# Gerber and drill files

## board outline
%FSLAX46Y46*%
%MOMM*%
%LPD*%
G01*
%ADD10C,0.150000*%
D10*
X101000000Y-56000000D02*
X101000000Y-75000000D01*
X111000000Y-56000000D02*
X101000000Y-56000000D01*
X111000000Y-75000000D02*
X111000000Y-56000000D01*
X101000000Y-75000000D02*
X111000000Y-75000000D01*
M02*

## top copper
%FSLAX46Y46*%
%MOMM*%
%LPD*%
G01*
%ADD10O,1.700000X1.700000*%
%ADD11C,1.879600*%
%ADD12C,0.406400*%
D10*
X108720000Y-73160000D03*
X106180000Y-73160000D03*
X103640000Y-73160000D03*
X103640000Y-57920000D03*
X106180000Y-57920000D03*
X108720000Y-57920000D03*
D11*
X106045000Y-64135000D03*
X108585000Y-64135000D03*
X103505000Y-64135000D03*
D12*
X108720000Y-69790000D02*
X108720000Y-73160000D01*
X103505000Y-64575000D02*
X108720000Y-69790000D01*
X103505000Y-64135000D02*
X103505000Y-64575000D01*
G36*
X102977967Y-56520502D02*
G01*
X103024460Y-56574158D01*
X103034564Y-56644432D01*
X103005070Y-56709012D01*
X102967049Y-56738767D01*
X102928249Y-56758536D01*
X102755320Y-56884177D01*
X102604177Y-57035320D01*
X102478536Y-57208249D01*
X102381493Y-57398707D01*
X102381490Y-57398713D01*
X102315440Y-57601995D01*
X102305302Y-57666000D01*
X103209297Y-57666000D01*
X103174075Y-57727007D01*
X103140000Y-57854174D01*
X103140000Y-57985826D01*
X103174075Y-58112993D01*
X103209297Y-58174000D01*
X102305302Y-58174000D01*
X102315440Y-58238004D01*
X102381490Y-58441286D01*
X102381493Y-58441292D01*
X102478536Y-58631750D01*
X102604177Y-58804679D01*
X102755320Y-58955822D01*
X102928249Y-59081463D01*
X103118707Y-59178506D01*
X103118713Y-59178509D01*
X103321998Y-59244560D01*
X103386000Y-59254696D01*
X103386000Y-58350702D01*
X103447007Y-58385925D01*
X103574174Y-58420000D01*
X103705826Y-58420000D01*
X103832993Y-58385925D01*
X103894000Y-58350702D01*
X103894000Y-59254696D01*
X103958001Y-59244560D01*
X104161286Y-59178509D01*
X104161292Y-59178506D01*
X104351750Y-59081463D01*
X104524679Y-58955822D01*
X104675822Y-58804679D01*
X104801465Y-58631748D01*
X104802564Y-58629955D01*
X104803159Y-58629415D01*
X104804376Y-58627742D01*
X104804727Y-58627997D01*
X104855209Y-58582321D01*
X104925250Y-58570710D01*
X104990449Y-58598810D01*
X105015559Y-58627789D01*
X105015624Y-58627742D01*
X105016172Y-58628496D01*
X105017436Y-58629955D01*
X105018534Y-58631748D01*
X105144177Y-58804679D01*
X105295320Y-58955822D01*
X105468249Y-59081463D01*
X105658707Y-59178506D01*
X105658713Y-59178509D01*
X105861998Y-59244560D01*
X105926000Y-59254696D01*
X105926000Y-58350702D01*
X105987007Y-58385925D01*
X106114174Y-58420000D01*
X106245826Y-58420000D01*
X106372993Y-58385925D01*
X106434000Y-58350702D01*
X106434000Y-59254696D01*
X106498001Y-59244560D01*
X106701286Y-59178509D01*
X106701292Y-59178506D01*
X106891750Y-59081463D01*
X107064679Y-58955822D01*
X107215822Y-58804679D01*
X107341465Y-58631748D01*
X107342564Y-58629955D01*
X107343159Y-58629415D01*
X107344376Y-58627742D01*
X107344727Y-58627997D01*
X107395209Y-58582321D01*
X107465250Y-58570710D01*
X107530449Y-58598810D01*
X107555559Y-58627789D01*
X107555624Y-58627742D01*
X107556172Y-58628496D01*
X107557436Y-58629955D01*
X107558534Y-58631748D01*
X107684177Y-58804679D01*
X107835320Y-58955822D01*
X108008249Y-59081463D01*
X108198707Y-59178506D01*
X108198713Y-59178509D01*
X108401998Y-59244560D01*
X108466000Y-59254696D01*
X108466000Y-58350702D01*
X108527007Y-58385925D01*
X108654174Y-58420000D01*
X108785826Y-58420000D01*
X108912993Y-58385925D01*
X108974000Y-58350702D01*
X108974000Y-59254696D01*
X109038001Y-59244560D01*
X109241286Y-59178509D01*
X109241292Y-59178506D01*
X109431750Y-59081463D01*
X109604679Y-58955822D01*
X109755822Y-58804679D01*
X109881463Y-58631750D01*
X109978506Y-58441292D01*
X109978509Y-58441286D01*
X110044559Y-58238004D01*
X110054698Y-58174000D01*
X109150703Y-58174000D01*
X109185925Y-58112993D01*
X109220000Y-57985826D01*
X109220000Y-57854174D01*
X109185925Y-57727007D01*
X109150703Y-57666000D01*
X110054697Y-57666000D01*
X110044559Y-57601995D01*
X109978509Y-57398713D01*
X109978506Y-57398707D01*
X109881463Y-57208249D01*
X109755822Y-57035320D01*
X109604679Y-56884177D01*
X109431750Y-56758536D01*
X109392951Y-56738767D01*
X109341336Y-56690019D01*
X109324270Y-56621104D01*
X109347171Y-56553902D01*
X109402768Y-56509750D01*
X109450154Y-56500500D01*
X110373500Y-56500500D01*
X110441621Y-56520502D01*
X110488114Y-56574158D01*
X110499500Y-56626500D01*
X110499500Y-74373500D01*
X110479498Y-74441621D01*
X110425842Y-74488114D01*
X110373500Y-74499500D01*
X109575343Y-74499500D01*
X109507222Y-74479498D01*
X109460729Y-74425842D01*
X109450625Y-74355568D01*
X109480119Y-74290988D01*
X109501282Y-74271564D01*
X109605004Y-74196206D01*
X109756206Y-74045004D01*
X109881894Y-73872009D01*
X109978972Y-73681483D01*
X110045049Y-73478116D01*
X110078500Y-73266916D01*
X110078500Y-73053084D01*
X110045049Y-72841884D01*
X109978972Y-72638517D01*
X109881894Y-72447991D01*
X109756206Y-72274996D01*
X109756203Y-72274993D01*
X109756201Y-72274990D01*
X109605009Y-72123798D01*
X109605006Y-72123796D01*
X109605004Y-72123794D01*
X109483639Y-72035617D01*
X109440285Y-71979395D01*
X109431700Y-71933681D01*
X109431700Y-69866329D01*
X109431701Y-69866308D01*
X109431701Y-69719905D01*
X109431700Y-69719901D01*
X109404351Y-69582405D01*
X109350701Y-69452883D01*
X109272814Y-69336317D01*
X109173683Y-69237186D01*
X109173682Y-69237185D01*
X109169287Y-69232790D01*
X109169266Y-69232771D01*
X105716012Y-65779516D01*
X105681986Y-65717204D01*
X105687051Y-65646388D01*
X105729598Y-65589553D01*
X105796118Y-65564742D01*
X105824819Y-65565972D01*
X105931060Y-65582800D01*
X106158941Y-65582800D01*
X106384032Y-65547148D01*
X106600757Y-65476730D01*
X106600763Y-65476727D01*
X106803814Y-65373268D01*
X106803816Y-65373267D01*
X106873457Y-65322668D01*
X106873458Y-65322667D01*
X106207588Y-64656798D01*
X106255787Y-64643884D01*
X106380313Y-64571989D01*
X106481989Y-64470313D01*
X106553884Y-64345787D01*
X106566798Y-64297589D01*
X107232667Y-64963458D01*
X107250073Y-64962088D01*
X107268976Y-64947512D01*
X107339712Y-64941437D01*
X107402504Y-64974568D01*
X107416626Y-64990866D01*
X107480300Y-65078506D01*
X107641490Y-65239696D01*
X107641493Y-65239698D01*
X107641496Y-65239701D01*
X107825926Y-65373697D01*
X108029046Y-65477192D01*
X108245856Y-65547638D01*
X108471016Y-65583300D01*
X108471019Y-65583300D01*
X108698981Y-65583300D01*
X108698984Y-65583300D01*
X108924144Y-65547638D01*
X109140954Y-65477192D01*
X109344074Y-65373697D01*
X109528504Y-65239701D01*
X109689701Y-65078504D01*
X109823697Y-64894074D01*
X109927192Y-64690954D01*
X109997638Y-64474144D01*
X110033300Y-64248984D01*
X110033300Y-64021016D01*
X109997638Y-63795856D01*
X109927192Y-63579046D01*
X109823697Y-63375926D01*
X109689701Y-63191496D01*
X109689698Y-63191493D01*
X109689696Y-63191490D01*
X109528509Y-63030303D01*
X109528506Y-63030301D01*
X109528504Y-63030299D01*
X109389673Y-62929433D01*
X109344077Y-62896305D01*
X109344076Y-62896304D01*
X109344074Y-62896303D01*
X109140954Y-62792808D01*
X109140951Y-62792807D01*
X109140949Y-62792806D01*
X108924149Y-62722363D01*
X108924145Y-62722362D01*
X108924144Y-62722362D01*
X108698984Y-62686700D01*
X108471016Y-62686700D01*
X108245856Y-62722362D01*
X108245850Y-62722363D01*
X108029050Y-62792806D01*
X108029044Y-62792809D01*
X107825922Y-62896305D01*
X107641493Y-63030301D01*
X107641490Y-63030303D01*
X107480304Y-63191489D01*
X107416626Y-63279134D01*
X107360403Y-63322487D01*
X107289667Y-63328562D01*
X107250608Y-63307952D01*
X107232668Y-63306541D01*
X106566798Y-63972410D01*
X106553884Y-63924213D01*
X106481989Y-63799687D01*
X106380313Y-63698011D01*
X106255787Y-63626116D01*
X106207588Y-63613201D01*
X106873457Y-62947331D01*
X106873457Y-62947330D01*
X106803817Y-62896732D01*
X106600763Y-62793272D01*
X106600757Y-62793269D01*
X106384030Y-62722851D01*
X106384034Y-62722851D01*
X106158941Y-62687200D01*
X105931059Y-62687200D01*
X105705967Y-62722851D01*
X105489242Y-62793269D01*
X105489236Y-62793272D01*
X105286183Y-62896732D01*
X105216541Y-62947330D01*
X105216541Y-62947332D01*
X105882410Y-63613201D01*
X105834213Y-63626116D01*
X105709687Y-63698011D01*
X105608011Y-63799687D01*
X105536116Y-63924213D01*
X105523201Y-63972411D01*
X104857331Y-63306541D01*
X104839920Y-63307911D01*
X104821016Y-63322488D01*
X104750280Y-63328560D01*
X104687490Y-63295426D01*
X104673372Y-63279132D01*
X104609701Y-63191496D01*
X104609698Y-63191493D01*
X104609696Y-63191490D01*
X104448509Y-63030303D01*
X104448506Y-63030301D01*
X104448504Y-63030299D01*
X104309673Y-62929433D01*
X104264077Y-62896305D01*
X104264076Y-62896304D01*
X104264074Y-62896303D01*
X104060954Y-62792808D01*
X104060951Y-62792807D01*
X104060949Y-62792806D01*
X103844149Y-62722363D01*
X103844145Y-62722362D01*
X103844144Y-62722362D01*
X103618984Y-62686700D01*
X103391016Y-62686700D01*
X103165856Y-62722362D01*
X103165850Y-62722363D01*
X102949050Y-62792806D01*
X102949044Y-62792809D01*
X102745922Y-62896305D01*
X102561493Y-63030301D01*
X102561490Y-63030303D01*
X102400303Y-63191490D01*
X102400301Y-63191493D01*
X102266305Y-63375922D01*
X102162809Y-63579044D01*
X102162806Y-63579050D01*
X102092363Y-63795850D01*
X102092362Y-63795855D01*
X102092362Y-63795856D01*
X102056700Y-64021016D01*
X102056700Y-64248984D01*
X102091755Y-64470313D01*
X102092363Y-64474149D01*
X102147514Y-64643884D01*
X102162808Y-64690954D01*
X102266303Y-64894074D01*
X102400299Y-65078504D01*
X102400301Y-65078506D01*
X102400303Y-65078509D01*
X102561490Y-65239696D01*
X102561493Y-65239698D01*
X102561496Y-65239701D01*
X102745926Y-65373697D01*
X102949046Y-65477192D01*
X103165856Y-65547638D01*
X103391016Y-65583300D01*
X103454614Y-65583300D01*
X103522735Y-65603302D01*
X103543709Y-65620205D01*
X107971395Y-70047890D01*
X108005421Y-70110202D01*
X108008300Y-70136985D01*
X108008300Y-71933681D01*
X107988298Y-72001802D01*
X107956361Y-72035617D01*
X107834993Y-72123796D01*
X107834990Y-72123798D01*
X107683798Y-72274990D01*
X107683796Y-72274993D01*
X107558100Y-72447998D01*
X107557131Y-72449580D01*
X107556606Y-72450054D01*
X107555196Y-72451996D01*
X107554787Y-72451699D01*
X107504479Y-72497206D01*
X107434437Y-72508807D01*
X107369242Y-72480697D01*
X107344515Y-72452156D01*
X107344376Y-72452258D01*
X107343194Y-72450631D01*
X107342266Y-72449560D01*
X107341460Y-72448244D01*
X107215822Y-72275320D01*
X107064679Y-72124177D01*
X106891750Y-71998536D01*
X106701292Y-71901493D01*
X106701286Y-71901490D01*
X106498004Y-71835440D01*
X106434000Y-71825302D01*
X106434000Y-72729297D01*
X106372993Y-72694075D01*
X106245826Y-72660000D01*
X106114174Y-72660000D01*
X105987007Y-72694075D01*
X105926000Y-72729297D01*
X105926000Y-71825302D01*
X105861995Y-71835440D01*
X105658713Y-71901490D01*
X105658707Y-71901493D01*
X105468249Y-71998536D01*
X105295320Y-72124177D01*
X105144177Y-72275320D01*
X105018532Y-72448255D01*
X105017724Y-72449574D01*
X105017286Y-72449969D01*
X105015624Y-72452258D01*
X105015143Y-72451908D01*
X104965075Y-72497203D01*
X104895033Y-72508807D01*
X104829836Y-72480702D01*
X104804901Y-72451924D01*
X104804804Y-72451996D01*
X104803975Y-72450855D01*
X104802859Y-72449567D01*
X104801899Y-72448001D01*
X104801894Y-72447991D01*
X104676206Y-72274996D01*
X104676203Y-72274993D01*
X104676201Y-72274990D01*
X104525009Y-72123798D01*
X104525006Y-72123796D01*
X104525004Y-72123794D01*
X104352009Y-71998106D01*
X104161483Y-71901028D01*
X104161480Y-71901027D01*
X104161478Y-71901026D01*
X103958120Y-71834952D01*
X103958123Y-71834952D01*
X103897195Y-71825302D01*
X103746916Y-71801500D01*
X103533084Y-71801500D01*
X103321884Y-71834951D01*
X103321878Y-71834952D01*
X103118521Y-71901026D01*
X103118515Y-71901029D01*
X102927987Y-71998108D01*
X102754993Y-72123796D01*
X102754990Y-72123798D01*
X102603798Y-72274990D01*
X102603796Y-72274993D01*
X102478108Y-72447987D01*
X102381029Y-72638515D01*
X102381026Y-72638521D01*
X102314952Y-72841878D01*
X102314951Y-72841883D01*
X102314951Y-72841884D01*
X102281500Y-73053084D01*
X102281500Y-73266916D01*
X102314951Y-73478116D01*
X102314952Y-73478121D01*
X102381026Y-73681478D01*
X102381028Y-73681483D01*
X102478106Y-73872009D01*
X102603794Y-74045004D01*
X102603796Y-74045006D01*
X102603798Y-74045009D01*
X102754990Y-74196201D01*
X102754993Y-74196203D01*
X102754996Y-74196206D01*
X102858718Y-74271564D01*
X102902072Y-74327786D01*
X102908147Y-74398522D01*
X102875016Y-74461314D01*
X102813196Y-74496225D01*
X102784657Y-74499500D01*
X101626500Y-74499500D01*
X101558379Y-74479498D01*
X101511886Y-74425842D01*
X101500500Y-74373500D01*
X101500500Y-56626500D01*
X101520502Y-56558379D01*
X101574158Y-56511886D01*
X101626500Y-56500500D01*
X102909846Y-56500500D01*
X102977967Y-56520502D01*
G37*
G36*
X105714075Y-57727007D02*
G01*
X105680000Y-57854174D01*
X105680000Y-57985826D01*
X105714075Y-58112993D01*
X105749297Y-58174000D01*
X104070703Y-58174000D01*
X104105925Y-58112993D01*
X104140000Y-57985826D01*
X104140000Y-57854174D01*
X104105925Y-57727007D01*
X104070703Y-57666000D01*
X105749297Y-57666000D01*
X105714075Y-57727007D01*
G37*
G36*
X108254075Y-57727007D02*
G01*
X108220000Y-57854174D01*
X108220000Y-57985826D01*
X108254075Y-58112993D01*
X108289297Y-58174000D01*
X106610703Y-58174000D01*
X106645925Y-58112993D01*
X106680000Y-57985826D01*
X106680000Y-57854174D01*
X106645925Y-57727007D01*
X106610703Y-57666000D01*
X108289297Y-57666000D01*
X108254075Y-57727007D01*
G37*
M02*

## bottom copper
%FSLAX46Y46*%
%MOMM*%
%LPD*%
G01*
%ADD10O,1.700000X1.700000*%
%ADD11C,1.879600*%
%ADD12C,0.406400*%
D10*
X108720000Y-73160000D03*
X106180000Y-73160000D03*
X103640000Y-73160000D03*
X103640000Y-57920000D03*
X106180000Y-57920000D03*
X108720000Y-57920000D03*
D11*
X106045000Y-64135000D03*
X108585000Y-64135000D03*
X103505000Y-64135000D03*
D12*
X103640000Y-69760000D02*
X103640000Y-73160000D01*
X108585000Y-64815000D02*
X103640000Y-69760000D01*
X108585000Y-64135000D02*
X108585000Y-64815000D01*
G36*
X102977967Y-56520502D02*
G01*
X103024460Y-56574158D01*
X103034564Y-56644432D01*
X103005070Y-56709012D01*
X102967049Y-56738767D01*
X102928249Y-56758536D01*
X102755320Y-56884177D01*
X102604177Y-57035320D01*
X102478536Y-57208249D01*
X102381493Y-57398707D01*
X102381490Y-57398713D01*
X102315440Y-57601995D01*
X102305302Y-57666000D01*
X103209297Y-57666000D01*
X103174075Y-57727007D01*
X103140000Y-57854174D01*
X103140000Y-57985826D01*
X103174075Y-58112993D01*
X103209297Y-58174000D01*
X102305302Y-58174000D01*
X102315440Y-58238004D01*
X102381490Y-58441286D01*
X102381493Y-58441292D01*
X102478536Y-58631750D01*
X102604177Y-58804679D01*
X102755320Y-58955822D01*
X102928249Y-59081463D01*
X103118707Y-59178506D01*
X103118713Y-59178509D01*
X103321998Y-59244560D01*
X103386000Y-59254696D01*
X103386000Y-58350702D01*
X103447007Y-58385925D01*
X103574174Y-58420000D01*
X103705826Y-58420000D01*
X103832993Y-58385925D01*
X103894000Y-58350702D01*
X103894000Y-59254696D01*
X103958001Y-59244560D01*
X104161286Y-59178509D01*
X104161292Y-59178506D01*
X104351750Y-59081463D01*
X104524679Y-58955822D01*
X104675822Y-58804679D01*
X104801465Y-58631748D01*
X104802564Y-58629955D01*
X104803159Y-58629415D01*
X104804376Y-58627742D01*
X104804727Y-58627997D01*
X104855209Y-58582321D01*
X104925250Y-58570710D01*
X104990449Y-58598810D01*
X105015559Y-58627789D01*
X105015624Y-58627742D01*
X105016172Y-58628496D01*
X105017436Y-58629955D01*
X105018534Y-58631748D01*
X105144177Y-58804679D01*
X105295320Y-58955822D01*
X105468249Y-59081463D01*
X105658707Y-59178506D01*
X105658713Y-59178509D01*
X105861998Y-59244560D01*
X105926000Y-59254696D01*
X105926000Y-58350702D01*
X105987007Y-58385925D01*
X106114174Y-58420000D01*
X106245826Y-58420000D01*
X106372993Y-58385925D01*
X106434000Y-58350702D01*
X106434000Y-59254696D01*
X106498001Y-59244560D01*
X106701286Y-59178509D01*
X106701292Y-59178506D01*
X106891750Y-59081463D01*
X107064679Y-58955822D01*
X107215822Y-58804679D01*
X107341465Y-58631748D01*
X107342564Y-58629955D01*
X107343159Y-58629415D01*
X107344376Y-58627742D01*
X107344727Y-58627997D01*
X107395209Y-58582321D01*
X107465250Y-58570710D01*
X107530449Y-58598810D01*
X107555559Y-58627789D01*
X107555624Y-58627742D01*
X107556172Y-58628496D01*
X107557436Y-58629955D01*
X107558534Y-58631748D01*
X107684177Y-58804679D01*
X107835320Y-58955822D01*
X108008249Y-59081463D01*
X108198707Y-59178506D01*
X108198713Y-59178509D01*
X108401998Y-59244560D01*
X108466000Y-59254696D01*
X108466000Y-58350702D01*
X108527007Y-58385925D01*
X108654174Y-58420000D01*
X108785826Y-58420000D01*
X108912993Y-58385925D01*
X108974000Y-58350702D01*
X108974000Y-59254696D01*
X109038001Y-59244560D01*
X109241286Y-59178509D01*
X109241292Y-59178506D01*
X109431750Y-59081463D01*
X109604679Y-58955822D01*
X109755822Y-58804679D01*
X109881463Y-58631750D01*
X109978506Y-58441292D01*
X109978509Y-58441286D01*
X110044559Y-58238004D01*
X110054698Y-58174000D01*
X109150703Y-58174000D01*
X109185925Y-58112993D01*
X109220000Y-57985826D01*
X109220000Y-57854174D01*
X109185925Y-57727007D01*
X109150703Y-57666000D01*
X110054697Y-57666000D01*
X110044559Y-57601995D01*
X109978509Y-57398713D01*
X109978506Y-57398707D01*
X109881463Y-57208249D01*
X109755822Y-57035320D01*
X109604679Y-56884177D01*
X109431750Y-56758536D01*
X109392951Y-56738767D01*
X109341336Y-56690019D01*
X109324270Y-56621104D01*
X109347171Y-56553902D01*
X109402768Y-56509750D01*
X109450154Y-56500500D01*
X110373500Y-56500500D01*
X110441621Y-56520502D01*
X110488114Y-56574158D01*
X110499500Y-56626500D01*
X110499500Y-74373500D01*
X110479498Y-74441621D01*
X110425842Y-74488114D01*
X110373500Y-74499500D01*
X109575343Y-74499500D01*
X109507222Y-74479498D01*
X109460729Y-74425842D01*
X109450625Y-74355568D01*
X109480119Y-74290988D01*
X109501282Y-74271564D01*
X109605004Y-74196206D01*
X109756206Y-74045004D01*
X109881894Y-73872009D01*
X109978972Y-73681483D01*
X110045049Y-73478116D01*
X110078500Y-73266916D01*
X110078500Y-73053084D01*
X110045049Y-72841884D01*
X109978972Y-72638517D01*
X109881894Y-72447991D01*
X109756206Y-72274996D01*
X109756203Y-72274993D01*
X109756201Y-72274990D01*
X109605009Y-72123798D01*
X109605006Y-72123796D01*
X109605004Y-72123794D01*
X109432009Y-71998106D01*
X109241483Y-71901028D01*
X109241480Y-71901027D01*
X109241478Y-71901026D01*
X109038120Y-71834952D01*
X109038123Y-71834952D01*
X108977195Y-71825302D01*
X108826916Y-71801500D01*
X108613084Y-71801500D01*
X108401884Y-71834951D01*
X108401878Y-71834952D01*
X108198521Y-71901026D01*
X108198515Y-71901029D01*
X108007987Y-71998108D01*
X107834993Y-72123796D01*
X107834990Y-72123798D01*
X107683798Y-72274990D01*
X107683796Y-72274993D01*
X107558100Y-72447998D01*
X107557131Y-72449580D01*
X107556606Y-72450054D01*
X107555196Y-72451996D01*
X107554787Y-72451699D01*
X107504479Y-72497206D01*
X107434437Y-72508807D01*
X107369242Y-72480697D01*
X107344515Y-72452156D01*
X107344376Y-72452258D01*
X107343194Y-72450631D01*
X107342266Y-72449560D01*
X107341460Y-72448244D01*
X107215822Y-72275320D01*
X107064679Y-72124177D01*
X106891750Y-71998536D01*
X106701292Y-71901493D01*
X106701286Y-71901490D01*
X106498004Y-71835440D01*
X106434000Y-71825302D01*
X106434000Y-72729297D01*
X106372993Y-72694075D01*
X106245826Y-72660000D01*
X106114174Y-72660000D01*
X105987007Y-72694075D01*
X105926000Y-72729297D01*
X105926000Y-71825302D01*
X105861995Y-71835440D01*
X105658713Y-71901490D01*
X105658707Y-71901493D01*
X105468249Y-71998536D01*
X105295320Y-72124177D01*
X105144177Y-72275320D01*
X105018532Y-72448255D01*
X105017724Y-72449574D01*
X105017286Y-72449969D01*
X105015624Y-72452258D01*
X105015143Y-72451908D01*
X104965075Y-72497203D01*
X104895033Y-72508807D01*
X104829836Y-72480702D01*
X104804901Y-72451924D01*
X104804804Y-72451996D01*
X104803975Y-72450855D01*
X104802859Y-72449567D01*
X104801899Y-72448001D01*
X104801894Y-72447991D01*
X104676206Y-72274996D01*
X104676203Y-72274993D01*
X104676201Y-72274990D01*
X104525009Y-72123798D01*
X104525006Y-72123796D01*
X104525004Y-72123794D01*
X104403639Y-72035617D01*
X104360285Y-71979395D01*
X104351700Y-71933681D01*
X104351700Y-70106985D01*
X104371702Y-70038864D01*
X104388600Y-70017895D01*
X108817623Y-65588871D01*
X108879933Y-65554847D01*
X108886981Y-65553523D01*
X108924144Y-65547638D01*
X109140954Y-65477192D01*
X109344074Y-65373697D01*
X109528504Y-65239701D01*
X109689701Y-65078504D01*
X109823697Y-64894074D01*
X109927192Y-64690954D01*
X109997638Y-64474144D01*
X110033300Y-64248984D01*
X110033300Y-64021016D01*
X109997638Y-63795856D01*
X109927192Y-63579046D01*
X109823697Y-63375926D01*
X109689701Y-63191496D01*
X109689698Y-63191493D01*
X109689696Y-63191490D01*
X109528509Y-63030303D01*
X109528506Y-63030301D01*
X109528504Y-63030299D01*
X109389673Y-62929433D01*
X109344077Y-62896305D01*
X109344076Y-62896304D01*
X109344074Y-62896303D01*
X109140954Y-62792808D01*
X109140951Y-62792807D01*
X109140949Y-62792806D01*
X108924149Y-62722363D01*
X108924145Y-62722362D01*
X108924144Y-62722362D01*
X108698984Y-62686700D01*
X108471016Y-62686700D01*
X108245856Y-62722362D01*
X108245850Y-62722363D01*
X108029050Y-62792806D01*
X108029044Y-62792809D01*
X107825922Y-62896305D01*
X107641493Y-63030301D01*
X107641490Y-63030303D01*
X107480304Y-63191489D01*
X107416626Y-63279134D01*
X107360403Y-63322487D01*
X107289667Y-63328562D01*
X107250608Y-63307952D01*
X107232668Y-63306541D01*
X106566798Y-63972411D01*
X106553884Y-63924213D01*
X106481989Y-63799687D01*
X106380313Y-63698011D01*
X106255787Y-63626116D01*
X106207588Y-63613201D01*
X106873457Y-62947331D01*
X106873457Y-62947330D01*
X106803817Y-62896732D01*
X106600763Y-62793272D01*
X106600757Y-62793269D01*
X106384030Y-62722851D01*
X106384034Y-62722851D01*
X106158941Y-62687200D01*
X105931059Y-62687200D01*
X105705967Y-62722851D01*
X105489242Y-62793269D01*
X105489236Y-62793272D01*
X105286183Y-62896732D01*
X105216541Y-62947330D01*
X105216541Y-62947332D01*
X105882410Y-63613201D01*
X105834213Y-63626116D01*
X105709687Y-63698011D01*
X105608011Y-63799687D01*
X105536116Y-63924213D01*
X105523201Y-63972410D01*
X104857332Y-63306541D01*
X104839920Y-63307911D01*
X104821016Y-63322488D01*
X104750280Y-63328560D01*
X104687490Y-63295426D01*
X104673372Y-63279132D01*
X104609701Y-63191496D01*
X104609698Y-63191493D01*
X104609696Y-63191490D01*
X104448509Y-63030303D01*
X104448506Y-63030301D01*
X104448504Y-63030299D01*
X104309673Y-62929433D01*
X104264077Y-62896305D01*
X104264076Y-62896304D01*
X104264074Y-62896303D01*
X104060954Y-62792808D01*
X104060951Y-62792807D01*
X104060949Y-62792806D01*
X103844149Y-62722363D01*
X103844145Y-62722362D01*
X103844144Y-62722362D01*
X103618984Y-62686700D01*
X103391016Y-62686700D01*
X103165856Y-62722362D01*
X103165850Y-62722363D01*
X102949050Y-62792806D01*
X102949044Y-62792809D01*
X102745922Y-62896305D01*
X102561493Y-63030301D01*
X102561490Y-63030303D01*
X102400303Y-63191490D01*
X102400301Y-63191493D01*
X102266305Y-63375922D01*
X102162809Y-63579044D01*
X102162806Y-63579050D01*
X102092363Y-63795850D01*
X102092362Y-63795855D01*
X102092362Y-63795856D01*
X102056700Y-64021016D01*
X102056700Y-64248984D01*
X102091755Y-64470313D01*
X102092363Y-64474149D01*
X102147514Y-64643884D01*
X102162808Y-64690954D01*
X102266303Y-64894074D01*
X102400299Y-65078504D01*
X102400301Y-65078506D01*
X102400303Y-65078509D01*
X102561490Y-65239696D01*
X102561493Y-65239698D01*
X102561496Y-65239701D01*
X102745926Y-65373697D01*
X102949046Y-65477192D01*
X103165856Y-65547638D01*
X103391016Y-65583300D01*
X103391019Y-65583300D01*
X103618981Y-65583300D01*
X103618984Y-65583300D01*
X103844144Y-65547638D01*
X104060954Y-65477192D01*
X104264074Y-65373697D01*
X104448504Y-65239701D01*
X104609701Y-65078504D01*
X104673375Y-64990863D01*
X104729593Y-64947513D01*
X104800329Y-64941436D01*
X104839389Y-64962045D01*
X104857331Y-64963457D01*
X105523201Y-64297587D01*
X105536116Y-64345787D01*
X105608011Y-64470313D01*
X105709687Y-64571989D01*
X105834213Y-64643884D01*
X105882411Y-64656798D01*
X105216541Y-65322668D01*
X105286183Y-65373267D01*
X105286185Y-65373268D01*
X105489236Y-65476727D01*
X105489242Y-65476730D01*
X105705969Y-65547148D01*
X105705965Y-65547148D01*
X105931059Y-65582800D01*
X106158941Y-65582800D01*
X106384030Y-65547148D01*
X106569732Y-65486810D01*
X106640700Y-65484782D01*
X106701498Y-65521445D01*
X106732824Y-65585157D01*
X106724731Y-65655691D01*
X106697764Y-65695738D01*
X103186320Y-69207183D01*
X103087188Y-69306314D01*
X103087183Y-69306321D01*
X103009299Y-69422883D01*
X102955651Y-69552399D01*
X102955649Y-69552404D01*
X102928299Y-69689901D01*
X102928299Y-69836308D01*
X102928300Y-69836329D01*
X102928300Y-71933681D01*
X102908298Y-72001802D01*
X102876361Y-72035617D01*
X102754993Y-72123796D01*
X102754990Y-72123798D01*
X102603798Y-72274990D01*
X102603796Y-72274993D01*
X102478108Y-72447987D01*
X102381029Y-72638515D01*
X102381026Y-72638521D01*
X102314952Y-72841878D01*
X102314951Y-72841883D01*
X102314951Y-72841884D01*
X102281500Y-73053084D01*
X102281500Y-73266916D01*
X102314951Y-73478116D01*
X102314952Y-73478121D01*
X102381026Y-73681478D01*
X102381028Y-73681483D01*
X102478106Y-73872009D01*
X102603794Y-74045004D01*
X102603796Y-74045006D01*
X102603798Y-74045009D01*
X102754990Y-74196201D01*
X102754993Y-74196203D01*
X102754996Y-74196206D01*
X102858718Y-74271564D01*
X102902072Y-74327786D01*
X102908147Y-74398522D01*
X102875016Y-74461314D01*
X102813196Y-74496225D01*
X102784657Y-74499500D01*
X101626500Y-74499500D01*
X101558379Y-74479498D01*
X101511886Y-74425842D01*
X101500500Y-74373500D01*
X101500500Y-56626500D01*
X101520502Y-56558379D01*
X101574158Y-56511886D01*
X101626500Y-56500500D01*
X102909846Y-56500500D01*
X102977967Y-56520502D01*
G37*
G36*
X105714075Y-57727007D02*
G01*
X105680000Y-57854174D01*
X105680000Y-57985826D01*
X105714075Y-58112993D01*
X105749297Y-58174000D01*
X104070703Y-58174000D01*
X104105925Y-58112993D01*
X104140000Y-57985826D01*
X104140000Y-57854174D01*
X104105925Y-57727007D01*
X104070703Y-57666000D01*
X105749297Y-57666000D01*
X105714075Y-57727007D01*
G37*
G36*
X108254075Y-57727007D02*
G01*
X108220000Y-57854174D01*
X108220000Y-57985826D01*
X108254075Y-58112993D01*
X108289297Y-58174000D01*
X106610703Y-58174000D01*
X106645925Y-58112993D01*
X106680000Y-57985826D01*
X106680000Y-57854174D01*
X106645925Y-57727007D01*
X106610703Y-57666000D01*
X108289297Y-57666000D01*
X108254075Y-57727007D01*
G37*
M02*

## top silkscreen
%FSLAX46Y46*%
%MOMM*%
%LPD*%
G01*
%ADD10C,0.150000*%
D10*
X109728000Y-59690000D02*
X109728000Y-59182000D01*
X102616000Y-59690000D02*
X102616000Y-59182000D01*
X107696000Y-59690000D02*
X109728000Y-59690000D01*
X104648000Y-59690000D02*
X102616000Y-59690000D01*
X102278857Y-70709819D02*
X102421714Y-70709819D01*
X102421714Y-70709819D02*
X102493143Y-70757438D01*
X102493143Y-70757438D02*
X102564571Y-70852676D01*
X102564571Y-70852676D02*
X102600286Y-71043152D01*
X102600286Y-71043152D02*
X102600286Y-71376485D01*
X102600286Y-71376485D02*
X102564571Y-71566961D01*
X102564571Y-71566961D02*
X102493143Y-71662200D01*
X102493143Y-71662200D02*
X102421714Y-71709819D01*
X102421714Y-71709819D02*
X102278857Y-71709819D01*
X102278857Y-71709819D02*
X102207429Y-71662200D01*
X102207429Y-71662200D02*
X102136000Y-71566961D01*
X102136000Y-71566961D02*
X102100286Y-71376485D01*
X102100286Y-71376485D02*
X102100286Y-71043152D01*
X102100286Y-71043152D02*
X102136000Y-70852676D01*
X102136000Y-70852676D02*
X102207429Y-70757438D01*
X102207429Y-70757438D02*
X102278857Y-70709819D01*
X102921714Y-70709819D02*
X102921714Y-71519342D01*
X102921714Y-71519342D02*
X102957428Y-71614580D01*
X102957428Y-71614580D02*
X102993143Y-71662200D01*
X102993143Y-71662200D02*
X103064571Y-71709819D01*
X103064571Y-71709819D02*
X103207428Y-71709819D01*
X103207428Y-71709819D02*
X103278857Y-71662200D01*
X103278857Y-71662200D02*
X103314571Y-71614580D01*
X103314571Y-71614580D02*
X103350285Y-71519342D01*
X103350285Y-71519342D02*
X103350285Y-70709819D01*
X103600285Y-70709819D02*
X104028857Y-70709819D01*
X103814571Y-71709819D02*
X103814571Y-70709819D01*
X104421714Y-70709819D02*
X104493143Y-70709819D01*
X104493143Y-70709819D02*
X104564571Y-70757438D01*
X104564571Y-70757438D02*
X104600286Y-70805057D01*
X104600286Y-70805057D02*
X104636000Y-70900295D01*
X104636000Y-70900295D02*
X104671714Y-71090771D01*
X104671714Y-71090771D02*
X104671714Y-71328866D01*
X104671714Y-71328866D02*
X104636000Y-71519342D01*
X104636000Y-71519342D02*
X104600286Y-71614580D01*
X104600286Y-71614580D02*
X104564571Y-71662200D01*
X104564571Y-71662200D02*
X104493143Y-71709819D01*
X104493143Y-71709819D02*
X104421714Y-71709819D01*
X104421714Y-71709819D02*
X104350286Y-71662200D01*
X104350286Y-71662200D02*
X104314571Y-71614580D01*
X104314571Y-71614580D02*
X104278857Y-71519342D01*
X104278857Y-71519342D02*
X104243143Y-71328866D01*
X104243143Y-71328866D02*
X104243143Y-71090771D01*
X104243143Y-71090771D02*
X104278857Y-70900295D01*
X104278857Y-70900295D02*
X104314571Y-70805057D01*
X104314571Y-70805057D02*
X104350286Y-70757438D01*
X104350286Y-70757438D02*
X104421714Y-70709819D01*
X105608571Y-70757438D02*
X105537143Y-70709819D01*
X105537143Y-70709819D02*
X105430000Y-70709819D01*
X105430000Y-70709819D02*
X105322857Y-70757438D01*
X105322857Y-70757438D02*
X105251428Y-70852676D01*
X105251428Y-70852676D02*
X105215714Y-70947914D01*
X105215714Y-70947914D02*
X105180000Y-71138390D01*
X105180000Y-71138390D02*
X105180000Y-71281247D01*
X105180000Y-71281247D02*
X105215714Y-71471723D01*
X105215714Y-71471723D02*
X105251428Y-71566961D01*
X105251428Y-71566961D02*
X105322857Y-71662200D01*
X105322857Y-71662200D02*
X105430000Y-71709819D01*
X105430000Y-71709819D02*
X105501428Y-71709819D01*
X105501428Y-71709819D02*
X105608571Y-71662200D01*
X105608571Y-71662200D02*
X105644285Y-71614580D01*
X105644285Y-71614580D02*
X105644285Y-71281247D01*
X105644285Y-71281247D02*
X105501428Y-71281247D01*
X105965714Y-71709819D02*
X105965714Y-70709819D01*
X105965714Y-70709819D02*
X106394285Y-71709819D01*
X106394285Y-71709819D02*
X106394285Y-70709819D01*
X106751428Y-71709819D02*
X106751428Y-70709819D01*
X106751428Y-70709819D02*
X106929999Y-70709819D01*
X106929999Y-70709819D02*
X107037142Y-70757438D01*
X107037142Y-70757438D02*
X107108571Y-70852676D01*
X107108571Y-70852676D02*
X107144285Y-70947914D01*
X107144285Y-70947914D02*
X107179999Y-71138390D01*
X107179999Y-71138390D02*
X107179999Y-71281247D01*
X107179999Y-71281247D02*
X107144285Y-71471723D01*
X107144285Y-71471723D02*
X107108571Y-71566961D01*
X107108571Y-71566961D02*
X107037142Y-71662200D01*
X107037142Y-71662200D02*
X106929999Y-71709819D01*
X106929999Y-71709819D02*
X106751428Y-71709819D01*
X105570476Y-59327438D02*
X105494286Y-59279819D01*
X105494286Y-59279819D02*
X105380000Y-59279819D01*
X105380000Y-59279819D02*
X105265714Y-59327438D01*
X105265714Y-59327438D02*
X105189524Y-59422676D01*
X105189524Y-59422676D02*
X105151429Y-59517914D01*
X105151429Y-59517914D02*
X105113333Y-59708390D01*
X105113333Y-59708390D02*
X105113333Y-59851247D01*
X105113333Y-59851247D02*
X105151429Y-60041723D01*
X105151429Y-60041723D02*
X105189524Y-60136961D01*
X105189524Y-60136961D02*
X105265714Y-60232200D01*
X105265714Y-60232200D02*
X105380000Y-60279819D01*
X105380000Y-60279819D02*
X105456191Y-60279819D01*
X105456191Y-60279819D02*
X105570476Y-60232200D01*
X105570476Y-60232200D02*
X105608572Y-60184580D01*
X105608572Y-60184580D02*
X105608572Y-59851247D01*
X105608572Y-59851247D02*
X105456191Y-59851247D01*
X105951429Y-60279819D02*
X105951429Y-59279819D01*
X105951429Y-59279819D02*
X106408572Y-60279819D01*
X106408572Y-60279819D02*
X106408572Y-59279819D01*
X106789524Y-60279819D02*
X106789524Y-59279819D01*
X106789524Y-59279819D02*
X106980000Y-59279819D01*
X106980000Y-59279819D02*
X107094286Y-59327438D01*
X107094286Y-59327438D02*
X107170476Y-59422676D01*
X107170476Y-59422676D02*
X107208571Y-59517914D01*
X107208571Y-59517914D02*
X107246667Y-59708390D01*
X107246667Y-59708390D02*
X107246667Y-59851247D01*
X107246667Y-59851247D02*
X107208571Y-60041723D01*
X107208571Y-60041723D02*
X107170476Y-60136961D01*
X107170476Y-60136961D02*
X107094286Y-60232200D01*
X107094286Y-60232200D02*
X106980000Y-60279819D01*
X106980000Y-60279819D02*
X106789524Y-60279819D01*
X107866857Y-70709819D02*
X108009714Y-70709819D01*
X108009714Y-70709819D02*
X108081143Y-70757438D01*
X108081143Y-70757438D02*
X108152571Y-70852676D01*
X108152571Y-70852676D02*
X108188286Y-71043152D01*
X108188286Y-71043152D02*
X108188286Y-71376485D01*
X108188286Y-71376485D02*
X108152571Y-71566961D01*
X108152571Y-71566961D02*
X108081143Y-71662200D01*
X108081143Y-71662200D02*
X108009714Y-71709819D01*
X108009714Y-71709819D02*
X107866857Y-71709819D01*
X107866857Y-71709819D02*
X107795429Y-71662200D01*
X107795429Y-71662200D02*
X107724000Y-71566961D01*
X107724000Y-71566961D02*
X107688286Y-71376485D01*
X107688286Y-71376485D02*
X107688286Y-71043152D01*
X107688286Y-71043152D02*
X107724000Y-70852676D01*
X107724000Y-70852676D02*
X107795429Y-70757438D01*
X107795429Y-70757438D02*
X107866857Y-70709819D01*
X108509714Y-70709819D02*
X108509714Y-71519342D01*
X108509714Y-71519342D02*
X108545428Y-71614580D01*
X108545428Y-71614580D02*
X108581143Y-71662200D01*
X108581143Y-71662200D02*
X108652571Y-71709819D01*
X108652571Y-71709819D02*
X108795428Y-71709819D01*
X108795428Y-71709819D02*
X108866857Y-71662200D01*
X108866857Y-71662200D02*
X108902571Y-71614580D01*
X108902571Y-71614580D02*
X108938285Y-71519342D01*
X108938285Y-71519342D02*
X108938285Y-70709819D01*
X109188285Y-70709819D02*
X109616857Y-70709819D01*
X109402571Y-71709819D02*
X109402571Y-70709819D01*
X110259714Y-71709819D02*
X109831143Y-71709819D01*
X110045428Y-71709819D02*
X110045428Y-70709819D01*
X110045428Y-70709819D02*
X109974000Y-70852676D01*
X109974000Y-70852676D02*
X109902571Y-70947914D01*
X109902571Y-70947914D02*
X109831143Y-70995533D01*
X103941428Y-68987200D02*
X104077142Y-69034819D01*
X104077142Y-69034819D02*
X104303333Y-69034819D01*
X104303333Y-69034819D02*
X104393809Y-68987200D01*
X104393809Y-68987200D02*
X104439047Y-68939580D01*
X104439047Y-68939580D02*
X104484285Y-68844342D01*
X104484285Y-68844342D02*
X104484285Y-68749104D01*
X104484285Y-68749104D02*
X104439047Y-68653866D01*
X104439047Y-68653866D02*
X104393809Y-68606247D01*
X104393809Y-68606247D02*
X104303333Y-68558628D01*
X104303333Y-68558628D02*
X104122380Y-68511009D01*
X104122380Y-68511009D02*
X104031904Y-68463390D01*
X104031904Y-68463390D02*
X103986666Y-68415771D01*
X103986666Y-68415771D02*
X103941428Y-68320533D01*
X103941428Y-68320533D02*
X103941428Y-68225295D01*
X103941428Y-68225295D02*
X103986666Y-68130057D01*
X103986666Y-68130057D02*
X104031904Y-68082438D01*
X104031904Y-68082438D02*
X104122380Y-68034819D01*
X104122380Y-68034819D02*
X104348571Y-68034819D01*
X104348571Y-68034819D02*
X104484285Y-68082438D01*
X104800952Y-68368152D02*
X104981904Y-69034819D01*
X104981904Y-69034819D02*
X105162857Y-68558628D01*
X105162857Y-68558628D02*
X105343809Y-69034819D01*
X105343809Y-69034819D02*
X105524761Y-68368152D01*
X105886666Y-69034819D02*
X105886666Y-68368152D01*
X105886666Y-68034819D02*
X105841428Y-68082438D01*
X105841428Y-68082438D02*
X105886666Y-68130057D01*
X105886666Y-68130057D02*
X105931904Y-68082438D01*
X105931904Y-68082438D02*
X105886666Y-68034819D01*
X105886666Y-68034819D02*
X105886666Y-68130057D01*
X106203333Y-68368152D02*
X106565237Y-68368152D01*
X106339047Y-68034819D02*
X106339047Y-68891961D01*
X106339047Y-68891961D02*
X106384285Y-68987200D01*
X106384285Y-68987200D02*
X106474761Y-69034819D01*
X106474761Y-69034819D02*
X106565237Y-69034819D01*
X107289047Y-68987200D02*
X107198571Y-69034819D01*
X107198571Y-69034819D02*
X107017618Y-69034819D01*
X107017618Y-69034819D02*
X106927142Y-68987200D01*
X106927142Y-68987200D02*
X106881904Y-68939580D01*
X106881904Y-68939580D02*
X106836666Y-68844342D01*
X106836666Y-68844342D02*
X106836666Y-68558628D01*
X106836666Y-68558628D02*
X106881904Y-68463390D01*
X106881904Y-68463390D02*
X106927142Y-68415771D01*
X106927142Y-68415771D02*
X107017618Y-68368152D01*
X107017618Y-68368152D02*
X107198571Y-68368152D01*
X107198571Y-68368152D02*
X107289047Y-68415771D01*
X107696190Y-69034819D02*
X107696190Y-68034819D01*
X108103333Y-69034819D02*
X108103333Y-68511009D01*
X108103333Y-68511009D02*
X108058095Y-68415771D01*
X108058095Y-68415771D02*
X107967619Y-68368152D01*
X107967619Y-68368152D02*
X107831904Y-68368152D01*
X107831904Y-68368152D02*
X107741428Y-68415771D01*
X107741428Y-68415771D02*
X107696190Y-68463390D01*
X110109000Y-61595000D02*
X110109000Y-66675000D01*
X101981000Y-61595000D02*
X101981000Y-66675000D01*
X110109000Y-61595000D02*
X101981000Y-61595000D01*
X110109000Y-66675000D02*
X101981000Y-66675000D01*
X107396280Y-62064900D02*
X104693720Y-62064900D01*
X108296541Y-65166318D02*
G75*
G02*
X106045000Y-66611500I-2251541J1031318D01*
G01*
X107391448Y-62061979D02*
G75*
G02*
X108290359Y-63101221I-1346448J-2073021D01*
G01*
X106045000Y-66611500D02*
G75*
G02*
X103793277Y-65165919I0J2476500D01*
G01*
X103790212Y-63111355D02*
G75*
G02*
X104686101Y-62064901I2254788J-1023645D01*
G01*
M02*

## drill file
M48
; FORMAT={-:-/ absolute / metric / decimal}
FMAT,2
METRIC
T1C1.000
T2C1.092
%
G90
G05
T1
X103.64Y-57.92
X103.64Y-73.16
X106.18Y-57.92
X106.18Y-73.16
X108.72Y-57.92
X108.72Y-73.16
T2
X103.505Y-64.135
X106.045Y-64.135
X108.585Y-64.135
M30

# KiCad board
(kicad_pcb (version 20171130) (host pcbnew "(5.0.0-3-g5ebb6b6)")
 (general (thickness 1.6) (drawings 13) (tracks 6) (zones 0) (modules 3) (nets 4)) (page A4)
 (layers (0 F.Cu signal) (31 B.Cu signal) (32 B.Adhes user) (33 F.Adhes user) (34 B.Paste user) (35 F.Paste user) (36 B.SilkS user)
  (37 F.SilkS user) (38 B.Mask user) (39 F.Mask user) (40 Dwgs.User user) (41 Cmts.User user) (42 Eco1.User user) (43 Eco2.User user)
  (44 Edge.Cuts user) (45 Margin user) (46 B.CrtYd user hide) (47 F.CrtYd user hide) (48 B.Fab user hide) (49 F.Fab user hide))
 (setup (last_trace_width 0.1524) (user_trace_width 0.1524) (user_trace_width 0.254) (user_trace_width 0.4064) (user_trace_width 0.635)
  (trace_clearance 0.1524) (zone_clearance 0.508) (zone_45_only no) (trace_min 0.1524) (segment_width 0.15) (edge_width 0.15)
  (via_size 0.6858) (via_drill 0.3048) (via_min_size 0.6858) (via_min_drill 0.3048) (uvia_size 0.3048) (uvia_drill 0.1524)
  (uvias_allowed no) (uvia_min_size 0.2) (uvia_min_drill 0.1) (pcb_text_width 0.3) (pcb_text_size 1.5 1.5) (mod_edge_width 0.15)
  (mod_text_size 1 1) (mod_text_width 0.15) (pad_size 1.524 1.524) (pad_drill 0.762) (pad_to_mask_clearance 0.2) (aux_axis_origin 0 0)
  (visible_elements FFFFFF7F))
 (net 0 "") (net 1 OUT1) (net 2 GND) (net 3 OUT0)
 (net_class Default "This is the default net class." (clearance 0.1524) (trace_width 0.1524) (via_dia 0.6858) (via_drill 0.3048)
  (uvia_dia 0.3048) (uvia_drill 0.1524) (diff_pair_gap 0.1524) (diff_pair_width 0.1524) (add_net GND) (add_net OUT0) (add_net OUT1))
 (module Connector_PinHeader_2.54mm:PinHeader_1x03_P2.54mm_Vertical (layer B.Cu) (at 103.64 73.16 270)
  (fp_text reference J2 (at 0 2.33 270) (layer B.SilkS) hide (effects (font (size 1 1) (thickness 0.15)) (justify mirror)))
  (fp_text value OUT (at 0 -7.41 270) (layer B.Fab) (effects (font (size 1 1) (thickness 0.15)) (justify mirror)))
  (pad 3 thru_hole oval (at 0 -5.08 270) (size 1.7 1.7) (drill 1) (layers *.Cu *.Mask) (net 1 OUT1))
  (pad 2 thru_hole oval (at 0 -2.54 270) (size 1.7 1.7) (drill 1) (layers *.Cu *.Mask) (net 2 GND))
  (pad 1 thru_hole oval (at 0 0 270) (size 1.7 1.7) (drill 1) (layers *.Cu *.Mask) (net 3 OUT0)))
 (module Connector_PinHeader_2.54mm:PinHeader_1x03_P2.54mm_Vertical (layer B.Cu) (at 103.64 57.92 270)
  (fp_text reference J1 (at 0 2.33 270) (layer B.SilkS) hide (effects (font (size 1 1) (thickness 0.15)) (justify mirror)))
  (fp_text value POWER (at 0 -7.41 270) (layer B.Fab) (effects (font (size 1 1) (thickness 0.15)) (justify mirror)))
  (pad 1 thru_hole oval (at 0 0 270) (size 1.7 1.7) (drill 1) (layers *.Cu *.Mask) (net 2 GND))
  (pad 2 thru_hole oval (at 0 -2.54 270) (size 1.7 1.7) (drill 1) (layers *.Cu *.Mask) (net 2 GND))
  (pad 3 thru_hole oval (at 0 -5.08 270) (size 1.7 1.7) (drill 1) (layers *.Cu *.Mask) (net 2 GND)))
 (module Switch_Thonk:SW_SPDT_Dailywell (layer F.Cu) (at 106.045 64.135 270)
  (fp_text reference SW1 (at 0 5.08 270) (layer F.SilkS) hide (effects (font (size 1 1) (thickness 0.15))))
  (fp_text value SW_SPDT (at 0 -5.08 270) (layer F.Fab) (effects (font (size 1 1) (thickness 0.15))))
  (fp_line (start -2.54 -4.064) (end 2.54 -4.064) (layer F.SilkS) (width 0.15))
  (fp_line (start -2.54 4.064) (end 2.54 4.064) (layer F.SilkS) (width 0.15))
  (fp_line (start -2.54 -4.064) (end -2.54 4.064) (layer F.SilkS) (width 0.15))
  (fp_line (start 2.54 -4.064) (end 2.54 4.064) (layer F.SilkS) (width 0.15))
  (fp_line (start -2.0701 -1.35128) (end -2.0701 1.35128) (layer F.SilkS) (width 0.15))
  (fp_arc (start 0 0) (end 2.4765 0) (angle -65.38985762) (layer F.SilkS) (width 0.15))
  (fp_arc (start 0 0) (end -1.033779 -2.245359) (angle -32.27419574) (layer F.SilkS) (width 0.15))
  (fp_arc (start 0 0) (end 2.4765 0) (angle 65.4) (layer F.SilkS) (width 0.15))
  (fp_arc (start 0 0) (end -2.070099 1.358899) (angle -32.3) (layer F.SilkS) (width 0.15))
  (pad 2 thru_hole circle (at 0 0 270) (size 1.8796 1.8796) (drill 1.0922) (layers *.Cu *.Mask) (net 2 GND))
  (pad 3 thru_hole circle (at 0 -2.54 270) (size 1.8796 1.8796) (drill 1.0922) (layers *.Cu *.Mask) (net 3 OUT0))
  (pad 1 thru_hole circle (at 0 2.54 270) (size 1.8796 1.8796) (drill 1.0922) (layers *.Cu *.Mask) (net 1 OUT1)))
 (gr_line (start 109.728 59.69) (end 109.728 59.182) (layer F.SilkS) (width 0.15))
 (gr_line (start 102.616 59.69) (end 102.616 59.182) (layer F.SilkS) (width 0.15))
 (gr_line (start 107.696 59.69) (end 109.728 59.69) (layer F.SilkS) (width 0.15))
 (gr_line (start 104.648 59.69) (end 102.616 59.69) (layer F.SilkS) (width 0.15))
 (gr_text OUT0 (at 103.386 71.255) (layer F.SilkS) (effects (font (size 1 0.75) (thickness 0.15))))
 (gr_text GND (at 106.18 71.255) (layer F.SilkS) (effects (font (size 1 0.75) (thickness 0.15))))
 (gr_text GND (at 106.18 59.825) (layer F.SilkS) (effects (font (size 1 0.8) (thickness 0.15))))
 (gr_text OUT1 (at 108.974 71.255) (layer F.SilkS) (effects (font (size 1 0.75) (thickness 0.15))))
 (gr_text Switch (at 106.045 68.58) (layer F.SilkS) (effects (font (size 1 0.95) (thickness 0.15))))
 (gr_line (start 101 56) (end 101 75) (layer Edge.Cuts) (width 0.15))
 (gr_line (start 111 56) (end 101 56) (layer Edge.Cuts) (width 0.15))
 (gr_line (start 111 75) (end 111 56) (layer Edge.Cuts) (width 0.15))
 (gr_line (start 101 75) (end 111 75) (layer Edge.Cuts) (width 0.15))
 (segment (start 108.72 69.79) (end 108.72 73.16) (width 0.4064) (layer F.Cu) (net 1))
 (segment (start 103.505 64.575) (end 108.72 69.79) (width 0.4064) (layer F.Cu) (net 1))
 (segment (start 103.505 64.135) (end 103.505 64.575) (width 0.4064) (layer F.Cu) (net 1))
 (segment (start 103.64 69.76) (end 103.64 73.16) (width 0.4064) (layer B.Cu) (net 3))
 (segment (start 108.585 64.815) (end 103.64 69.76) (width 0.4064) (layer B.Cu) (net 3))
 (segment (start 108.585 64.135) (end 108.585 64.815) (width 0.4064) (layer B.Cu) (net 3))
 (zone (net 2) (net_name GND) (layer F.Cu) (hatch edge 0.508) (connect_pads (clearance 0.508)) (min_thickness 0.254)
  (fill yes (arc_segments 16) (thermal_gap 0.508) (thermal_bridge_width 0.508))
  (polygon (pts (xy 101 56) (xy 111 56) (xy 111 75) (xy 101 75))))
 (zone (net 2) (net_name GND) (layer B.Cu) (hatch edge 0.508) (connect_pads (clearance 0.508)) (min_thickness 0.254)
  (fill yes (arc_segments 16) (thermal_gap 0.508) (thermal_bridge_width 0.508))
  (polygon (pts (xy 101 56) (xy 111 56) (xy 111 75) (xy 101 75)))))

